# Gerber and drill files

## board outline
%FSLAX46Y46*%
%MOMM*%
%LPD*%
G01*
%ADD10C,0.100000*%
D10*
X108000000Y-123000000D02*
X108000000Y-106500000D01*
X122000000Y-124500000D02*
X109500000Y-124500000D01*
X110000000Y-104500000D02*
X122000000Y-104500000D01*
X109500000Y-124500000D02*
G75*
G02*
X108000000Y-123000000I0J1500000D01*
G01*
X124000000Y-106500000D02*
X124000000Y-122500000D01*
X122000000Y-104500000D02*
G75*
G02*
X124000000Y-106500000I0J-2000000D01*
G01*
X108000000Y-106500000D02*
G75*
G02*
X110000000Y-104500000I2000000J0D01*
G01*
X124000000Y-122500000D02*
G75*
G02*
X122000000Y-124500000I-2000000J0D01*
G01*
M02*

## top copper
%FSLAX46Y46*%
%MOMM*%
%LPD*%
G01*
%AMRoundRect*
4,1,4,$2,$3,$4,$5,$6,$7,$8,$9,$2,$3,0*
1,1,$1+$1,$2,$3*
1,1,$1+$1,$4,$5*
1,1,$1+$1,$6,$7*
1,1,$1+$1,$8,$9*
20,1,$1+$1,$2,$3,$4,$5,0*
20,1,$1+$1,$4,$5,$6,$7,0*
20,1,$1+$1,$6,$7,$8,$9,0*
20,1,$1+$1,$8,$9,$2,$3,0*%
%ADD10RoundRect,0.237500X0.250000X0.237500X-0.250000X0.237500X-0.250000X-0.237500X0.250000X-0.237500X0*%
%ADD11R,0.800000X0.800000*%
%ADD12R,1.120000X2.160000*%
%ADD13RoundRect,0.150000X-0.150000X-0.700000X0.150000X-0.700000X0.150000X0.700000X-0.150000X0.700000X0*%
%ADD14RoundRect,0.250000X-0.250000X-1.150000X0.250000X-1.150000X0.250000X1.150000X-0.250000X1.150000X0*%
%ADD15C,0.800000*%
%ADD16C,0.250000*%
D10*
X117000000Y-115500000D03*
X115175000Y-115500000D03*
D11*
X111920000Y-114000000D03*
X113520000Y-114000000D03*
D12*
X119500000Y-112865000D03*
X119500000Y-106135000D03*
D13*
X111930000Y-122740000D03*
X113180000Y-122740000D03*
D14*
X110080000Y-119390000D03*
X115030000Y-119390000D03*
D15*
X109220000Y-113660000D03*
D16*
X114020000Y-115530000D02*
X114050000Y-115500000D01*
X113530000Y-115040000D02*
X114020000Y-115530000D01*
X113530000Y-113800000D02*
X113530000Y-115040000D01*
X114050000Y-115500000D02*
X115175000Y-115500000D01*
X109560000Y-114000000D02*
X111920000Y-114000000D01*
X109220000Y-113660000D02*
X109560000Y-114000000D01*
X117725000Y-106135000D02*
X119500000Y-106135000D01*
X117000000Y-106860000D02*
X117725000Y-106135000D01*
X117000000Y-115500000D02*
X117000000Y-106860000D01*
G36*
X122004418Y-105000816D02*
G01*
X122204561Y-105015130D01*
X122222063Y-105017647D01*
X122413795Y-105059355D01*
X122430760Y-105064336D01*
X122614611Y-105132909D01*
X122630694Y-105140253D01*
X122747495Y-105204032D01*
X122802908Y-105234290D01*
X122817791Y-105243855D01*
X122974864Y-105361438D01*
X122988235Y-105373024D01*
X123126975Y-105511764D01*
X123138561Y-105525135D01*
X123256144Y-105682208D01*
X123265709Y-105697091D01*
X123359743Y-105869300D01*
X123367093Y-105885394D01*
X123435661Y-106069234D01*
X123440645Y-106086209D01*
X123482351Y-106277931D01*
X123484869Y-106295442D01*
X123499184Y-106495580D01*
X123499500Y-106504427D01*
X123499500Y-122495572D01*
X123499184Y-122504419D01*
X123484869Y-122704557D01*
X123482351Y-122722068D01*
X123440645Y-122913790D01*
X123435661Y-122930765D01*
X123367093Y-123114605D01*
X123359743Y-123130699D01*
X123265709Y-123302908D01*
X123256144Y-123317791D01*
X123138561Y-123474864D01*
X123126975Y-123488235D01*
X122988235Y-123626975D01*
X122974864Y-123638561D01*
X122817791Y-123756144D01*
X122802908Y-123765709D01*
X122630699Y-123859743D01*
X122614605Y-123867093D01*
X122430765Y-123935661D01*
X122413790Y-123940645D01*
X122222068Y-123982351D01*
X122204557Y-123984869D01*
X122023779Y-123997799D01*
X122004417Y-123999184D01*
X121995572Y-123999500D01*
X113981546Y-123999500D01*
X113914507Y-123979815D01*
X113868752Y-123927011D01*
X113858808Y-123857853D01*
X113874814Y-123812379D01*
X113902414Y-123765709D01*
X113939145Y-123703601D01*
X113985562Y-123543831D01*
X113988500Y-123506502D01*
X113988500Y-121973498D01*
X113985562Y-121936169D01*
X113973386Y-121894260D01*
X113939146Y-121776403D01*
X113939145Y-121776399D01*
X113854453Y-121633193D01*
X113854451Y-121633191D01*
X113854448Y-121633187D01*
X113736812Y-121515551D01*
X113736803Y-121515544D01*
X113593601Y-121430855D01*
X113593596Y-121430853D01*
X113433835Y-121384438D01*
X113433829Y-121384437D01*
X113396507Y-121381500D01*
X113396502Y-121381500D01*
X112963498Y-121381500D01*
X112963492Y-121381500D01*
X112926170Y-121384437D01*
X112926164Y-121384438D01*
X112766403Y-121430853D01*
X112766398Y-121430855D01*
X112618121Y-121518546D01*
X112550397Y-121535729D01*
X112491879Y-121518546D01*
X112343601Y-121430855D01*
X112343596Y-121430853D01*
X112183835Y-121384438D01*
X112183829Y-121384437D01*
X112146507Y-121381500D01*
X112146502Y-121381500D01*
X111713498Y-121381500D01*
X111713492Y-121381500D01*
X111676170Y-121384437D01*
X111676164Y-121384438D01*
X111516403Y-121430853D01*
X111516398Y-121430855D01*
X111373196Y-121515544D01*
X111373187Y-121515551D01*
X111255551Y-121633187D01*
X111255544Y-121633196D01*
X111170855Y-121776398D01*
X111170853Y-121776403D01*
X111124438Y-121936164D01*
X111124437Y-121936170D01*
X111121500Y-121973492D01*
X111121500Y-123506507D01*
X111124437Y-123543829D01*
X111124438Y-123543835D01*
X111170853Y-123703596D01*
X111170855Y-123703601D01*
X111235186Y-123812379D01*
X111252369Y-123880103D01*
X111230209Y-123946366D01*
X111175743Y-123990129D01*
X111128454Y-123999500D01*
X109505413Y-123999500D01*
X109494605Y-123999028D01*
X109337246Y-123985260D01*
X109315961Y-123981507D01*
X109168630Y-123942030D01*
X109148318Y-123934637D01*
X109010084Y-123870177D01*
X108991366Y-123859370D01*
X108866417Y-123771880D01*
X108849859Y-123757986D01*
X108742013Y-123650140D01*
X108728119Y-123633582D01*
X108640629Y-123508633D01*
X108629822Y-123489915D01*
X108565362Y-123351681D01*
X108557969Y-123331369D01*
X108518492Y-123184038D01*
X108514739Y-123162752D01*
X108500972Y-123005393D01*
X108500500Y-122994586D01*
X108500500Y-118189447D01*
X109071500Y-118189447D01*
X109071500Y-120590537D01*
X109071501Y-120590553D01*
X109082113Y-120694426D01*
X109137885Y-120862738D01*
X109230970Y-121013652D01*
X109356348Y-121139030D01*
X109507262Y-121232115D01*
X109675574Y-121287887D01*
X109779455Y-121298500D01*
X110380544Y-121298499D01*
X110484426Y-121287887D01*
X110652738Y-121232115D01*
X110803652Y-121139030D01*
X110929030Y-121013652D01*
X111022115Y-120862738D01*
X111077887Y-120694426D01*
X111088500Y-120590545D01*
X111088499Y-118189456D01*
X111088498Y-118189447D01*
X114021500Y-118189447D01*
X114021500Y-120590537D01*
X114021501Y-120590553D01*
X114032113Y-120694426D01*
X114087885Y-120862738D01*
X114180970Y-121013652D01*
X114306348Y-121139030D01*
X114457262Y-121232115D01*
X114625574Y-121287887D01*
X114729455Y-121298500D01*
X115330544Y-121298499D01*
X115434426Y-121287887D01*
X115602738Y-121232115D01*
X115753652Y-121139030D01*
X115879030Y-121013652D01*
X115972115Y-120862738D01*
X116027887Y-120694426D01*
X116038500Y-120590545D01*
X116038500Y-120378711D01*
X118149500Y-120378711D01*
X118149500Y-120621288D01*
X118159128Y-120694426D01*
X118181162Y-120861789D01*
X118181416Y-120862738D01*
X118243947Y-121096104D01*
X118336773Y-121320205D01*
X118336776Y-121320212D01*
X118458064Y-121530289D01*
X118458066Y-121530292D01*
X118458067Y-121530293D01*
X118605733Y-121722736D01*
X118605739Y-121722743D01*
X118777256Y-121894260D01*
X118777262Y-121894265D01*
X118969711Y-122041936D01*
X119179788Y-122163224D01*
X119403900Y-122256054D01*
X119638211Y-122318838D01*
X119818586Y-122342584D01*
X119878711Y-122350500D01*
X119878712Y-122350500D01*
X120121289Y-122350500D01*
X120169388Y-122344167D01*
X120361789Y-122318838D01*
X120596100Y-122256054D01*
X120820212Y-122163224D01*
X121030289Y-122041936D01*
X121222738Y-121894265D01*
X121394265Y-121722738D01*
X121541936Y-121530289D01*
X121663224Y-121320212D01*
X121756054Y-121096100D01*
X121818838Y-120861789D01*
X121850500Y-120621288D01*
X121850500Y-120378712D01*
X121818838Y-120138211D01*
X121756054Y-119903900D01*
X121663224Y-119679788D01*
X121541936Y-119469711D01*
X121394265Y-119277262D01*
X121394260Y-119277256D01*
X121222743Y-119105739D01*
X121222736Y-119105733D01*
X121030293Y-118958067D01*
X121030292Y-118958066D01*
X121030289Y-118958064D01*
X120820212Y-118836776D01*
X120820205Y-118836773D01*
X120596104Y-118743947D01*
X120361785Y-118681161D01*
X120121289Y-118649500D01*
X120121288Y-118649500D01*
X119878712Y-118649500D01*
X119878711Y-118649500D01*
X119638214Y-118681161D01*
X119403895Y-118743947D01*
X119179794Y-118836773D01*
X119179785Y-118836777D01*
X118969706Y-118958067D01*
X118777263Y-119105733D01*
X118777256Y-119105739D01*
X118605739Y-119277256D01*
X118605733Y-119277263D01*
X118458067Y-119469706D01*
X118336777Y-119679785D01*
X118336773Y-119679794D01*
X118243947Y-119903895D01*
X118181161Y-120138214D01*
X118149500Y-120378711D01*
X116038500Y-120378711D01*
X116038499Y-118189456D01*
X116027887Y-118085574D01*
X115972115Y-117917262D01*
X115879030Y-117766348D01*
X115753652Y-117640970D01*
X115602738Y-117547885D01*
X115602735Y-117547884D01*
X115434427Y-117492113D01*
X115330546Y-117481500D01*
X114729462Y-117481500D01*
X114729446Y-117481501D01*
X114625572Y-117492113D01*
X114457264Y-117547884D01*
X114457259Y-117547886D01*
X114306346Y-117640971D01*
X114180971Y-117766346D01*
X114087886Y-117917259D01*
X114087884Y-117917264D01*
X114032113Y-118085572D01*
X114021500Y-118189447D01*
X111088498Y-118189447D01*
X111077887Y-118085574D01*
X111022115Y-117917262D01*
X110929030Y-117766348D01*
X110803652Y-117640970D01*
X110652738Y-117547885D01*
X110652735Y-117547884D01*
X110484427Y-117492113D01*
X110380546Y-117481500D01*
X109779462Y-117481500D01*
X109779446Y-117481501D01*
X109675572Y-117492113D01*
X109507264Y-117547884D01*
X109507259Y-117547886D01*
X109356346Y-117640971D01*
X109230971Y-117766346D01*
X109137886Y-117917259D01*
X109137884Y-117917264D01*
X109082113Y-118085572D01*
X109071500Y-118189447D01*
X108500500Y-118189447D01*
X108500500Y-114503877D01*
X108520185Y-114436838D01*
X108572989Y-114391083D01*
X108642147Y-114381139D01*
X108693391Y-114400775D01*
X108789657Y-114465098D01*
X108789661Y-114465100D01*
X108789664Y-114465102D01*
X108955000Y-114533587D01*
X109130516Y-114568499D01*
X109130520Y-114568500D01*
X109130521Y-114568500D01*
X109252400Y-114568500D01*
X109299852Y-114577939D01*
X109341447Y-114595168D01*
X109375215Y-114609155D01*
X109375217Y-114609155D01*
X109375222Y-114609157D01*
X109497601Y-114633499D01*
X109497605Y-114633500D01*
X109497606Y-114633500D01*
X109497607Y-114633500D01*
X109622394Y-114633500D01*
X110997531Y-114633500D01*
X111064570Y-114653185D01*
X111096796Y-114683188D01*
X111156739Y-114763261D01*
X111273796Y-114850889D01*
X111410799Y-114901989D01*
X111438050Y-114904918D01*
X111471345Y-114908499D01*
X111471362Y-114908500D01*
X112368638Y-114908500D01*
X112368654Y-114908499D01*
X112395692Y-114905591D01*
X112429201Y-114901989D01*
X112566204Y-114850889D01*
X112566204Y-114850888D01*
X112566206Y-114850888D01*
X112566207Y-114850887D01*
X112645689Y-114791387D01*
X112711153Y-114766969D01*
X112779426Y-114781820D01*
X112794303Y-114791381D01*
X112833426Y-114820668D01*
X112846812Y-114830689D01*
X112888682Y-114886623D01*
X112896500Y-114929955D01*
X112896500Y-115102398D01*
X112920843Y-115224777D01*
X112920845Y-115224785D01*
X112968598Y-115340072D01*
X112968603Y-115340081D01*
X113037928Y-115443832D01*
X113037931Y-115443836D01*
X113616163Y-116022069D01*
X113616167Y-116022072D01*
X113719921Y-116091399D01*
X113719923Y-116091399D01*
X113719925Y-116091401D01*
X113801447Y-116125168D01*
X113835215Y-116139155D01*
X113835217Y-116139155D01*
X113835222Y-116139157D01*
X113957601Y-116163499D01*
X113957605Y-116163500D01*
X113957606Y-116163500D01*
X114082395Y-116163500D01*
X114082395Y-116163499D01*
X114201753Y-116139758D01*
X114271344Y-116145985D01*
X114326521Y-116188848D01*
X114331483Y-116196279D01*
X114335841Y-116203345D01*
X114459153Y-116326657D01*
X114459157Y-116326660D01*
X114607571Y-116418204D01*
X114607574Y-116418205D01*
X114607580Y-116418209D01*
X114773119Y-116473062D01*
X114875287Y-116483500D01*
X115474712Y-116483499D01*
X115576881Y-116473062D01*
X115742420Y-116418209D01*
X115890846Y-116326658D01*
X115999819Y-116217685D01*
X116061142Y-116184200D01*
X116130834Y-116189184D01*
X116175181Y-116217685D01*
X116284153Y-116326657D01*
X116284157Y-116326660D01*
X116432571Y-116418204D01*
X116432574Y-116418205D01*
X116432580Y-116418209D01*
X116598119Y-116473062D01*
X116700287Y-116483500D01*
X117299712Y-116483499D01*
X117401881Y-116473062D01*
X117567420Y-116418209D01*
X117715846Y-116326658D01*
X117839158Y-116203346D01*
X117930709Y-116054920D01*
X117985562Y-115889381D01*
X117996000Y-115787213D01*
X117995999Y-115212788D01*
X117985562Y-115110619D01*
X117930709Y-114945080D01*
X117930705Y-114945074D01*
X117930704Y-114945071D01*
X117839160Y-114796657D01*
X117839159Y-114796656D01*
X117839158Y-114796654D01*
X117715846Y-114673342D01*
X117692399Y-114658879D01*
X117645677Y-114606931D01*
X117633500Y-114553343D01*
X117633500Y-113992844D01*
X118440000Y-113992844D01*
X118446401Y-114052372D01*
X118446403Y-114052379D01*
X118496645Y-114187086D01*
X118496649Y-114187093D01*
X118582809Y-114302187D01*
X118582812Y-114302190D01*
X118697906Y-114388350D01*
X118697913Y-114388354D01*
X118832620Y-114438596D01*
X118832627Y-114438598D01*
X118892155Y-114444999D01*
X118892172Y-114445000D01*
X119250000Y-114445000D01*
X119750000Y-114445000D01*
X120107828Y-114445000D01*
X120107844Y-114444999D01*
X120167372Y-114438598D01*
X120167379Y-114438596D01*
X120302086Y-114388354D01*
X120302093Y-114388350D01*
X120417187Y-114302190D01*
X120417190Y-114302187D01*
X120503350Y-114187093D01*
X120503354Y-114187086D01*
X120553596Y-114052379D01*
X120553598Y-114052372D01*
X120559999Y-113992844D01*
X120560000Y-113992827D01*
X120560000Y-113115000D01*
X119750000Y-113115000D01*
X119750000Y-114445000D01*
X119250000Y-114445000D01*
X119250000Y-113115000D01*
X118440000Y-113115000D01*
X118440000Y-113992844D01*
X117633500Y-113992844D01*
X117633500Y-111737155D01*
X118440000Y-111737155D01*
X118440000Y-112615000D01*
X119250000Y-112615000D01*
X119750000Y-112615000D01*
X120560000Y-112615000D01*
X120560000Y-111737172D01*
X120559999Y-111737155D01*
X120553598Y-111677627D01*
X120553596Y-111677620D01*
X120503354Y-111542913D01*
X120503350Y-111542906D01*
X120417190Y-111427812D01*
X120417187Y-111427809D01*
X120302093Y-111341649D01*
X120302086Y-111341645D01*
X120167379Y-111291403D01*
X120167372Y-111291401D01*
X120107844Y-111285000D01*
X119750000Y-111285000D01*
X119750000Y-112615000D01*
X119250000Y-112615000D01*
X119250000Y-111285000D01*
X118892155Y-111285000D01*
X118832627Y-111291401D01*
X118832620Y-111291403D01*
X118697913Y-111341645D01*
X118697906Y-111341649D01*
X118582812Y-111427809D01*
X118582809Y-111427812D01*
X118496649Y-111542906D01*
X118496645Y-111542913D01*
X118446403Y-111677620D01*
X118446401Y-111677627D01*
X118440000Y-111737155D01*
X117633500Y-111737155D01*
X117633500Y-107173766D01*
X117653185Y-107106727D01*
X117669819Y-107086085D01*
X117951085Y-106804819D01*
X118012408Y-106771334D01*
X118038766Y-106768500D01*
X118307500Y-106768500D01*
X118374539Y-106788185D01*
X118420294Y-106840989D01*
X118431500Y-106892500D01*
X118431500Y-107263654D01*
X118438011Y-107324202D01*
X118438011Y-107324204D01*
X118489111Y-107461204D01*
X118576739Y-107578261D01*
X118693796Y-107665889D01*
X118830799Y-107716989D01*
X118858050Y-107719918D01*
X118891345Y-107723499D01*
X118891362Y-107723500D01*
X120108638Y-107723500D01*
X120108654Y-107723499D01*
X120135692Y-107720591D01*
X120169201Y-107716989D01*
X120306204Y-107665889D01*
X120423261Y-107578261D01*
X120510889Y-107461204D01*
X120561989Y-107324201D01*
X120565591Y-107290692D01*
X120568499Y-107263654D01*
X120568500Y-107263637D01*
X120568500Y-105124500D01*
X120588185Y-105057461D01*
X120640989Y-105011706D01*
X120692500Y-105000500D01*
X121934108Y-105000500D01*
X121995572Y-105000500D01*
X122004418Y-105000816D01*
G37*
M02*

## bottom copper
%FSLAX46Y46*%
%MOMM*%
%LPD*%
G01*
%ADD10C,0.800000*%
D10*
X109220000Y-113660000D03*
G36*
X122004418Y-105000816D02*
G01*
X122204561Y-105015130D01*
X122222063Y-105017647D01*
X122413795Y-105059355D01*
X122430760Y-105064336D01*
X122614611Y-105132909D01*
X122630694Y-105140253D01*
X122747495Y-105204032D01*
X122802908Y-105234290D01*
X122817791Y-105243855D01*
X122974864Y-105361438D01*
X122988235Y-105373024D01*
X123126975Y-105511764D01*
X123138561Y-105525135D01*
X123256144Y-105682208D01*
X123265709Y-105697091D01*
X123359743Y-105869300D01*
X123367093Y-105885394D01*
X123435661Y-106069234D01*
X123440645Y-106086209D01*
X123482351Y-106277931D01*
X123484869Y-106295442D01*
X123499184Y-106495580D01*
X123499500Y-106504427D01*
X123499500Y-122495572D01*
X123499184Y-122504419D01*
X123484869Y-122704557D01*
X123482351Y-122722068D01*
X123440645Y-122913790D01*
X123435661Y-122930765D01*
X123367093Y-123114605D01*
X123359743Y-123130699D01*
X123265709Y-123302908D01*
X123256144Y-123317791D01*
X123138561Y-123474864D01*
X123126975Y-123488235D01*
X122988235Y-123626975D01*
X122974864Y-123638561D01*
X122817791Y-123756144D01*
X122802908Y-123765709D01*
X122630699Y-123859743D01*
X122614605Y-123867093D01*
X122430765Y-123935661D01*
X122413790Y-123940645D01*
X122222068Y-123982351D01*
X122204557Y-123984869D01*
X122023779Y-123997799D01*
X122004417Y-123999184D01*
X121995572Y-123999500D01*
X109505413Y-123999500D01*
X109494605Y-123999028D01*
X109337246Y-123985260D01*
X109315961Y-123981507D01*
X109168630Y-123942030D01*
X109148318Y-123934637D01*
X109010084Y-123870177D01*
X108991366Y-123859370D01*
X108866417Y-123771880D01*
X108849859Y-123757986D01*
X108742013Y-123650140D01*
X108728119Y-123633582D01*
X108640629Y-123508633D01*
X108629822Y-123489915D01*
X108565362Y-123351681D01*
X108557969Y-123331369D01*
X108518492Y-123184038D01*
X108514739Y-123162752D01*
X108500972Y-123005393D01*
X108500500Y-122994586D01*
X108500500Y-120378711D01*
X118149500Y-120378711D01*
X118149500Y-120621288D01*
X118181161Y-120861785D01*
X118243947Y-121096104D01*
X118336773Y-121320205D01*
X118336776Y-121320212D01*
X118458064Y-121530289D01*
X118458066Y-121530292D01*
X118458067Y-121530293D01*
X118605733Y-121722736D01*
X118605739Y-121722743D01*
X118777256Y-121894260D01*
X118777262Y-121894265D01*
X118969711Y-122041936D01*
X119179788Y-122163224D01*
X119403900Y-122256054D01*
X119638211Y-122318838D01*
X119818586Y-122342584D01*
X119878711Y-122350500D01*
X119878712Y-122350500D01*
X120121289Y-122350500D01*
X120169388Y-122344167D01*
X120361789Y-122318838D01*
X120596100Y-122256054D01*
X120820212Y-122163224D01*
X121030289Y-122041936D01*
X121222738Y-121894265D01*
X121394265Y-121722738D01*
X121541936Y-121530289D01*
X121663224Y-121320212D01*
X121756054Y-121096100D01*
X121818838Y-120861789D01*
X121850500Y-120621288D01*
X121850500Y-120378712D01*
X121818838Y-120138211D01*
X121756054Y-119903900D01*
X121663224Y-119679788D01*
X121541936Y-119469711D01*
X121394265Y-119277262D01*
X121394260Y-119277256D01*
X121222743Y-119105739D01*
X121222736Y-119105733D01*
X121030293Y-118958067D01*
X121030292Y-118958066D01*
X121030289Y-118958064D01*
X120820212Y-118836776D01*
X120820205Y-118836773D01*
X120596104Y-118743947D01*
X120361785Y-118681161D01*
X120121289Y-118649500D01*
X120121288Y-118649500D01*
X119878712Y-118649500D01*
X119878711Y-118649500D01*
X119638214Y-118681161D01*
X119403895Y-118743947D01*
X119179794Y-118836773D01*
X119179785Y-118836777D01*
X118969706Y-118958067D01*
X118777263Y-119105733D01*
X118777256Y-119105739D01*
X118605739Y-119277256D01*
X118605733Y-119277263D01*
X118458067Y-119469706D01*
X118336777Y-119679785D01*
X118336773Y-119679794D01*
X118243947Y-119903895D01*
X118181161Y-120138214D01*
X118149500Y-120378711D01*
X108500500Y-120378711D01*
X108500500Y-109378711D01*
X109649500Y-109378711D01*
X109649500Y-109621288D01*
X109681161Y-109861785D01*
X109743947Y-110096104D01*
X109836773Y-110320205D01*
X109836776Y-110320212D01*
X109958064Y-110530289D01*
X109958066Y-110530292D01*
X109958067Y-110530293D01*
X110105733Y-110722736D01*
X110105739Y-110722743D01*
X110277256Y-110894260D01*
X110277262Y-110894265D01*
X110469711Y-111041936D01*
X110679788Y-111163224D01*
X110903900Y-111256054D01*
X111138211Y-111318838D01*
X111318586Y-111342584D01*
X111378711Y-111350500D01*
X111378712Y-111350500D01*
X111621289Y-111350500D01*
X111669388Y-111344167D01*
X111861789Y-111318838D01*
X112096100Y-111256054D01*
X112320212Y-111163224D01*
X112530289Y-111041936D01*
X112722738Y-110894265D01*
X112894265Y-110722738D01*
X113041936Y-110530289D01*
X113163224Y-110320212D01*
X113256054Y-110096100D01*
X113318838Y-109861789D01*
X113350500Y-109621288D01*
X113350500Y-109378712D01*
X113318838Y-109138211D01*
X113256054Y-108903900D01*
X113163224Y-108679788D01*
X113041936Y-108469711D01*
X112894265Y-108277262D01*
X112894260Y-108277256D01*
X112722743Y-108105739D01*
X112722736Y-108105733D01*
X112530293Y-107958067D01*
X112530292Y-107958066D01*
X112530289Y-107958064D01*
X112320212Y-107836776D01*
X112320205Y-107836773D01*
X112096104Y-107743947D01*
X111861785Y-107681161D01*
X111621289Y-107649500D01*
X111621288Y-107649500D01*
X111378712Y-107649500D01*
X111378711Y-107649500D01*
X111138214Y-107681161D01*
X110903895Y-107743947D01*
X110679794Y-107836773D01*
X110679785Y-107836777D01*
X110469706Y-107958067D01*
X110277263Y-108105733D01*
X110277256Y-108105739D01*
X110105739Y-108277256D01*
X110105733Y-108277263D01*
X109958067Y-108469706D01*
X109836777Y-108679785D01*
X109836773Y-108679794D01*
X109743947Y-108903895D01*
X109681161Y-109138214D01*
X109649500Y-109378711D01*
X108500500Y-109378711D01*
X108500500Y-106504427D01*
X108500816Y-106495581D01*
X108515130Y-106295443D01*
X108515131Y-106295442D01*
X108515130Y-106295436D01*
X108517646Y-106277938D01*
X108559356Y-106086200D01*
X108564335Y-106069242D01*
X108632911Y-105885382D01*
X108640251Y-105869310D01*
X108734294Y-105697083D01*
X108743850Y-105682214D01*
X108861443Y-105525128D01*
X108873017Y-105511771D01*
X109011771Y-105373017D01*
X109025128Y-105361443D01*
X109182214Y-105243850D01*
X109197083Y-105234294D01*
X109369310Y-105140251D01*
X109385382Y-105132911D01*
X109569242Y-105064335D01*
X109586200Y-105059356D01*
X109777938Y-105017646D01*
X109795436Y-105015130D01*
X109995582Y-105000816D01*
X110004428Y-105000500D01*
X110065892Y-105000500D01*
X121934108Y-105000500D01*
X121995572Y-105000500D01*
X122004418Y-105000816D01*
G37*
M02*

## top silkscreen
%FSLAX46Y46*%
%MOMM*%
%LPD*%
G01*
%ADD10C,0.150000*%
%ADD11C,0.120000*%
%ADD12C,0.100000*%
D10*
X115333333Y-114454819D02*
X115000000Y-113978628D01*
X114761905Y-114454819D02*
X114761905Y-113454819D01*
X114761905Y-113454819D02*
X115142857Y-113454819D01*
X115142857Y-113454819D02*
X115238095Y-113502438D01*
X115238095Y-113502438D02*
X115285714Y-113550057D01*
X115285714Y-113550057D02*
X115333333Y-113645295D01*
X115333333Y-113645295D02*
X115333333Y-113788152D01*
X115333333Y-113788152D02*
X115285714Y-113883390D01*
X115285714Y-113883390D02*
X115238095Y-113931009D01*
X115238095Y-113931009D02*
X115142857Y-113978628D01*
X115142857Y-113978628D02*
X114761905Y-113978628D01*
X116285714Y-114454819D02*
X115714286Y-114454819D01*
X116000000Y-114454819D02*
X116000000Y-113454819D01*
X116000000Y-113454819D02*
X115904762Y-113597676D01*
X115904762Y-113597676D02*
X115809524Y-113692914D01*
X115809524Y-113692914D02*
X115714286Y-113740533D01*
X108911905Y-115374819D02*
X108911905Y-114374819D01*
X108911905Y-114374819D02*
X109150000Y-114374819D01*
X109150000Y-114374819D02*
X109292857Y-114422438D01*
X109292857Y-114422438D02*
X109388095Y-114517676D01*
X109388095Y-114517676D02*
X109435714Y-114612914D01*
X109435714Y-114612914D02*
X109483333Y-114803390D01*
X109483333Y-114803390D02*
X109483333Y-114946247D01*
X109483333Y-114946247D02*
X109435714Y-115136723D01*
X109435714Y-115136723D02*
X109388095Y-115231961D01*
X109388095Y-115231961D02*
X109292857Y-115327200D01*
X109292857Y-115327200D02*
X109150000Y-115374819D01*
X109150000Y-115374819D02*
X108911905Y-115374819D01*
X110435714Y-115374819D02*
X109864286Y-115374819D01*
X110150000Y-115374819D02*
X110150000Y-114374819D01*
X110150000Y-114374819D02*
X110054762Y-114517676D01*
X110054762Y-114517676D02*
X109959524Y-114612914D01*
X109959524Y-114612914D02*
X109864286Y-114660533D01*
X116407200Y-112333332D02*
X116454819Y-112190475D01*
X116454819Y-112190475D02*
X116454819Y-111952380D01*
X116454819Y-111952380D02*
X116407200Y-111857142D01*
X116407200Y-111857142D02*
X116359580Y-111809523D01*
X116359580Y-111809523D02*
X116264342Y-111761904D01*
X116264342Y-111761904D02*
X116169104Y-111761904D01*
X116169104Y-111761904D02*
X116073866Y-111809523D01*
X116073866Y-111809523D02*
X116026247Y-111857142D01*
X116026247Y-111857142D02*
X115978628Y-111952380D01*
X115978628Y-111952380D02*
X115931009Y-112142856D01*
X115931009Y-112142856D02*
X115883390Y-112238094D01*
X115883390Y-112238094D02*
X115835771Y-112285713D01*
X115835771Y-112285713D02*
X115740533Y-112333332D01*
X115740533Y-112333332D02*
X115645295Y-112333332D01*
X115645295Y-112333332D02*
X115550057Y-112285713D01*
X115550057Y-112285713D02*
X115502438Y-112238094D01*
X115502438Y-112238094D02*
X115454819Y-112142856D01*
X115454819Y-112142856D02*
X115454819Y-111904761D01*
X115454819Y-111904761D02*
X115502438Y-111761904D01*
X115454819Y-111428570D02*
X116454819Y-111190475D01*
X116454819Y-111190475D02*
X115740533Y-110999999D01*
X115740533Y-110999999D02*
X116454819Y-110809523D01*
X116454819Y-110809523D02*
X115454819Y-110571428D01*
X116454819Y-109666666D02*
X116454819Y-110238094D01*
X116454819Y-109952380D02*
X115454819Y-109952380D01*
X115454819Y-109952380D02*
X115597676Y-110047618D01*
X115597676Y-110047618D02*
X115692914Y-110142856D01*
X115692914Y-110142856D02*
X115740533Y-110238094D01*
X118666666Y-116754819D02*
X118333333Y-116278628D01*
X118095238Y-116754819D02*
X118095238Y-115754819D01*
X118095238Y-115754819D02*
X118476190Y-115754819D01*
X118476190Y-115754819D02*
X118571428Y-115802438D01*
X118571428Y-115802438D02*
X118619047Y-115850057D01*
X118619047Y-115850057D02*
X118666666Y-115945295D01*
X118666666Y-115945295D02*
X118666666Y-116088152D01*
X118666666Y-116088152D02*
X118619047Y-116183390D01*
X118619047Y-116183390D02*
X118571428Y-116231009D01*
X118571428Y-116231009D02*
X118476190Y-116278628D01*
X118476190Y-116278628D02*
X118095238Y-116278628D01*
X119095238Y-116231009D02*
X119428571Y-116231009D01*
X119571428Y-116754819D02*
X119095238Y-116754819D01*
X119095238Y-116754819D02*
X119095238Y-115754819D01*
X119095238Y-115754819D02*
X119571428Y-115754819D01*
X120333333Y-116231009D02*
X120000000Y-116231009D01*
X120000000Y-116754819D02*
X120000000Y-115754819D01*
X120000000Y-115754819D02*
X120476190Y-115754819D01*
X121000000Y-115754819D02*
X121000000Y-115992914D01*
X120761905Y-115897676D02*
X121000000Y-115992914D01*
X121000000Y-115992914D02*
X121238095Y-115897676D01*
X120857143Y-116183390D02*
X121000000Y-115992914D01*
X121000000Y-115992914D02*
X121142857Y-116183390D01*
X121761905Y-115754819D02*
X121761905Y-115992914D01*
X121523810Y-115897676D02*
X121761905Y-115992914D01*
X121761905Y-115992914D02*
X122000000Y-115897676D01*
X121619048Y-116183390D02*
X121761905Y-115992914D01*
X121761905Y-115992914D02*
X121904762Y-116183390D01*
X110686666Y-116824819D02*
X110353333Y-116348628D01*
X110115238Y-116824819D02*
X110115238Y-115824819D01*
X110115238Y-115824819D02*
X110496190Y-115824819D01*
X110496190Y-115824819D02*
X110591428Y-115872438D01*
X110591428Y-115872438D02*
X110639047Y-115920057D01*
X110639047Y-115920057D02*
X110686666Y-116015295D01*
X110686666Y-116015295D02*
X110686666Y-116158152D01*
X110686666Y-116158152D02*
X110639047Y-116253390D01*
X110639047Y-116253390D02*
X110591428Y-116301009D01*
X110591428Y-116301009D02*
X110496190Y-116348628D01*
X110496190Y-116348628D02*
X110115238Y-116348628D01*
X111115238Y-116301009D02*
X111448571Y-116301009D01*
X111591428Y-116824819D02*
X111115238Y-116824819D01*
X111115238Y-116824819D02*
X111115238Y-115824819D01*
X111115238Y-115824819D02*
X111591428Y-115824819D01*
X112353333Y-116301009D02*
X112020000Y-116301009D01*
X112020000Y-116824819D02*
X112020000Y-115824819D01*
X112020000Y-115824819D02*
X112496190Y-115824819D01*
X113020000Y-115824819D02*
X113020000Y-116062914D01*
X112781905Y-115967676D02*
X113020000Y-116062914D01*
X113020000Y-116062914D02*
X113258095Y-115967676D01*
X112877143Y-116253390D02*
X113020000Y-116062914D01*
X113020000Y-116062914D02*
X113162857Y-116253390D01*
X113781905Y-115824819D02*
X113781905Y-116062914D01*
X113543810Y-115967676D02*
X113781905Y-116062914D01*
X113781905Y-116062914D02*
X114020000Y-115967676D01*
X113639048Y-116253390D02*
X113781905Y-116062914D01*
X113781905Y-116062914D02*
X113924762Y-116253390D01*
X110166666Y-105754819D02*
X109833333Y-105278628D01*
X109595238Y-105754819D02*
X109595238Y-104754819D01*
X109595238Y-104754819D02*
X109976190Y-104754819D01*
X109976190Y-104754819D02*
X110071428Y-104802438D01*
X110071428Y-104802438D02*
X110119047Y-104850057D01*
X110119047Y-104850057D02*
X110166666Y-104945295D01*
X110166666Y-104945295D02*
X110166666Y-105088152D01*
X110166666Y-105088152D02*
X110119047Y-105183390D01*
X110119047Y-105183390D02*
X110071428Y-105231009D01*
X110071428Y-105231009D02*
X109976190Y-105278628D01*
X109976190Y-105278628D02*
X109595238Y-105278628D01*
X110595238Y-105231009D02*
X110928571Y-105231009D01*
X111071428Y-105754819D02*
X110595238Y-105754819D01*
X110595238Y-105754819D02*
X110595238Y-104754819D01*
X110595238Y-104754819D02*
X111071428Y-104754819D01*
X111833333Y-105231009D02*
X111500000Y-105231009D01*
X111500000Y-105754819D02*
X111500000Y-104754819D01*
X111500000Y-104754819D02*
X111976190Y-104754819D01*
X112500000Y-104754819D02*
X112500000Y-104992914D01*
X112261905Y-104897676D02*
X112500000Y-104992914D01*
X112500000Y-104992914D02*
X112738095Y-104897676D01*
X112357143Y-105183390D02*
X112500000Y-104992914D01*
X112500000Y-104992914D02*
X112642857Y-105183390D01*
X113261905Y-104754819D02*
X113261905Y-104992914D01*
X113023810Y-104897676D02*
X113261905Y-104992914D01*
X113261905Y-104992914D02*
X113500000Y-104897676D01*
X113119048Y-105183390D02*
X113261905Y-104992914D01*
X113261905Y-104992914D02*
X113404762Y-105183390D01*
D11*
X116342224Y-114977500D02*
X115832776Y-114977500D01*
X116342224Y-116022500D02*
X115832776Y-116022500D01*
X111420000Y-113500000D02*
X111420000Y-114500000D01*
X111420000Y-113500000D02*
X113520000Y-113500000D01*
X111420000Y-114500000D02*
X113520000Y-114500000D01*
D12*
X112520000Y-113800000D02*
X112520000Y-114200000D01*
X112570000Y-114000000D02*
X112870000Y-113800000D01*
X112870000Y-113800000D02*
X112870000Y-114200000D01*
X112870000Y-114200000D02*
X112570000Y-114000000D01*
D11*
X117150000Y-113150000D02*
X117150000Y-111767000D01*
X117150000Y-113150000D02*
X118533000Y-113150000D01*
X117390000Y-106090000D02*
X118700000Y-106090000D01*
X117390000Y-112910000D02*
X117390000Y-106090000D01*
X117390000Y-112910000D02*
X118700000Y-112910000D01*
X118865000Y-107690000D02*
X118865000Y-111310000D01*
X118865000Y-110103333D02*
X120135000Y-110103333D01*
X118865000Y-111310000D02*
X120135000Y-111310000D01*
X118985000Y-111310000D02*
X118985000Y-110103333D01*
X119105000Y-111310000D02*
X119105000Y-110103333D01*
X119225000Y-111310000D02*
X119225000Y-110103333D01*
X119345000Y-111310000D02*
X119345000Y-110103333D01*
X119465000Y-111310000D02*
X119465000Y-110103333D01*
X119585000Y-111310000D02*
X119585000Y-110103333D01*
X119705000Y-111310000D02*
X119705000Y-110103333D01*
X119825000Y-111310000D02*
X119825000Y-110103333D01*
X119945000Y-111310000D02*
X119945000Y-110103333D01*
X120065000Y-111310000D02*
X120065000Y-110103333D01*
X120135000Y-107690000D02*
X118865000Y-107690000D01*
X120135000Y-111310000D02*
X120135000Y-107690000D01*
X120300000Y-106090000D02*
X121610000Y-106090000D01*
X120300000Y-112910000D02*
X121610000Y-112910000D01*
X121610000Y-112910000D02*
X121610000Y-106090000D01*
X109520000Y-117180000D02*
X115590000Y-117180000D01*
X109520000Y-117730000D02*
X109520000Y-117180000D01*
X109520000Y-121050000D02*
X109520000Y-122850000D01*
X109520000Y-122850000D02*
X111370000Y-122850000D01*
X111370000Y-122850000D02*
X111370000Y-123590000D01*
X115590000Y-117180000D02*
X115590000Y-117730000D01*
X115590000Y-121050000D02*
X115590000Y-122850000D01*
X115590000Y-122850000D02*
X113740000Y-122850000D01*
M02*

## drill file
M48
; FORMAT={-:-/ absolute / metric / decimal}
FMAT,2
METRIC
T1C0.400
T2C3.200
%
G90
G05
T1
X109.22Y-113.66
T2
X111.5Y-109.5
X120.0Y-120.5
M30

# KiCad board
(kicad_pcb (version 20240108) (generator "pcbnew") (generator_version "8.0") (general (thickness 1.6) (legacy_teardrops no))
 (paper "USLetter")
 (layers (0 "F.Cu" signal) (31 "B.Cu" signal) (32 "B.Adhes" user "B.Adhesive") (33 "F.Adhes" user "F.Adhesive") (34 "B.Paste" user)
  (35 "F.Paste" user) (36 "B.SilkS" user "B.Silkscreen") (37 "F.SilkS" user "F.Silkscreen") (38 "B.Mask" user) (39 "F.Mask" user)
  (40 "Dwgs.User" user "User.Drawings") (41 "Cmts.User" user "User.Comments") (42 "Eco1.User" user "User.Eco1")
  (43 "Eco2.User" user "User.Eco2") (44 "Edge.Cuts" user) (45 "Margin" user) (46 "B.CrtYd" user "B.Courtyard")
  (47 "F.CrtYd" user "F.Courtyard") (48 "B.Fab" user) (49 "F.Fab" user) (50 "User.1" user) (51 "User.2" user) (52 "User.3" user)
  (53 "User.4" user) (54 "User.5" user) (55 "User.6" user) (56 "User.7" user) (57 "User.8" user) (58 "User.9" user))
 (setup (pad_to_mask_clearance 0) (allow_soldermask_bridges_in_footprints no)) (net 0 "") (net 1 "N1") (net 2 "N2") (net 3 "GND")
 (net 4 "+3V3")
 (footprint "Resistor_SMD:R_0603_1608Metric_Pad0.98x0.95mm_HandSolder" (layer "F.Cu") (at 116.0875 115.5 180)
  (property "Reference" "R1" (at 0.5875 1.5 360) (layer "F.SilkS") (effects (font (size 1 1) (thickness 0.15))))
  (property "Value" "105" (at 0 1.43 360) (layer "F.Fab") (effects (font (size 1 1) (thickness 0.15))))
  (fp_line (start -0.254724 0.5225) (end 0.254724 0.5225) (stroke (width 0.12) (type solid)) (layer "F.SilkS"))
  (fp_line (start -0.254724 -0.5225) (end 0.254724 -0.5225) (stroke (width 0.12) (type solid)) (layer "F.SilkS"))
  (pad "1" smd roundrect (at -0.9125 0 180) (size 0.975 0.95) (layers "F.Cu" "F.Paste" "F.Mask") (roundrect_rratio 0.25) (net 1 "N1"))
  (pad "2" smd roundrect (at 0.9125 0 180) (size 0.975 0.95) (layers "F.Cu" "F.Paste" "F.Mask") (roundrect_rratio 0.25) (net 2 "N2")))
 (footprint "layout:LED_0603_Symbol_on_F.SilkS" (layer "F.Cu") (at 112.72 114)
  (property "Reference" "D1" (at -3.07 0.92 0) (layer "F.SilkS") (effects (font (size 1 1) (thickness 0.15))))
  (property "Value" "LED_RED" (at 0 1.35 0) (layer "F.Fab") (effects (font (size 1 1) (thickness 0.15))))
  (fp_line (start -1.3 -0.5) (end -1.3 0.5) (stroke (width 0.12) (type solid)) (layer "F.SilkS"))
  (fp_line (start -1.3 -0.5) (end 0.8 -0.5) (stroke (width 0.12) (type solid)) (layer "F.SilkS"))
  (fp_line (start -1.3 0.5) (end 0.8 0.5) (stroke (width 0.12) (type solid)) (layer "F.SilkS"))
  (fp_line (start -0.2 -0.2) (end -0.2 0.2) (stroke (width 0.1) (type solid)) (layer "F.SilkS"))
  (fp_line (start -0.15 0) (end 0.15 -0.2) (stroke (width 0.1) (type solid)) (layer "F.SilkS"))
  (fp_line (start 0.15 -0.2) (end 0.15 0.2) (stroke (width 0.1) (type solid)) (layer "F.SilkS"))
  (fp_line (start 0.15 0.2) (end -0.15 0) (stroke (width 0.1) (type solid)) (layer "F.SilkS"))
  (pad "1" smd rect (at -0.8 0 180) (size 0.8 0.8) (layers "F.Cu" "F.Paste" "F.Mask") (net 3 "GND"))
  (pad "2" smd rect (at 0.8 0 180) (size 0.8 0.8) (layers "F.Cu" "F.Paste" "F.Mask") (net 2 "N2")))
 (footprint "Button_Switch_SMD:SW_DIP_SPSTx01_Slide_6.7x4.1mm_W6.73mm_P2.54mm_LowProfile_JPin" (layer "F.Cu") (at 119.5 109.5 90)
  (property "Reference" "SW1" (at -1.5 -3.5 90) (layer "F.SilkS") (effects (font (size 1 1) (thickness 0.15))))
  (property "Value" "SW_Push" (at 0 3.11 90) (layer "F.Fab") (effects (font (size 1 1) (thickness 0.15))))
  (fp_line (start -3.65 -2.35) (end -2.267 -2.35) (stroke (width 0.12) (type solid)) (layer "F.SilkS"))
  (fp_line (start -3.65 -2.35) (end -3.65 -0.967) (stroke (width 0.12) (type solid)) (layer "F.SilkS"))
  (fp_line (start 3.41 -2.11) (end 3.41 -0.8) (stroke (width 0.12) (type solid)) (layer "F.SilkS"))
  (fp_line (start -3.41 -2.11) (end 3.41 -2.11) (stroke (width 0.12) (type solid)) (layer "F.SilkS"))
  (fp_line (start -3.41 -2.11) (end -3.41 -0.8) (stroke (width 0.12) (type solid)) (layer "F.SilkS"))
  (fp_line (start 1.81 -0.635) (end -1.81 -0.635) (stroke (width 0.12) (type solid)) (layer "F.SilkS"))
  (fp_line (start -0.603333 -0.635) (end -0.603333 0.635) (stroke (width 0.12) (type solid)) (layer "F.SilkS"))
  (fp_line (start -1.81 -0.635) (end -1.81 0.635) (stroke (width 0.12) (type solid)) (layer "F.SilkS"))
  (fp_line (start -1.81 -0.515) (end -0.603333 -0.515) (stroke (width 0.12) (type solid)) (layer "F.SilkS"))
  (fp_line (start -1.81 -0.395) (end -0.603333 -0.395) (stroke (width 0.12) (type solid)) (layer "F.SilkS"))
  (fp_line (start -1.81 -0.275) (end -0.603333 -0.275) (stroke (width 0.12) (type solid)) (layer "F.SilkS"))
  (fp_line (start -1.81 -0.155) (end -0.603333 -0.155) (stroke (width 0.12) (type solid)) (layer "F.SilkS"))
  (fp_line (start -1.81 -0.035) (end -0.603333 -0.035) (stroke (width 0.12) (type solid)) (layer "F.SilkS"))
  (fp_line (start -1.81 0.085) (end -0.603333 0.085) (stroke (width 0.12) (type solid)) (layer "F.SilkS"))
  (fp_line (start -1.81 0.205) (end -0.603333 0.205) (stroke (width 0.12) (type solid)) (layer "F.SilkS"))
  (fp_line (start -1.81 0.325) (end -0.603333 0.325) (stroke (width 0.12) (type solid)) (layer "F.SilkS"))
  (fp_line (start -1.81 0.445) (end -0.603333 0.445) (stroke (width 0.12) (type solid)) (layer "F.SilkS"))
  (fp_line (start -1.81 0.565) (end -0.603333 0.565) (stroke (width 0.12) (type solid)) (layer "F.SilkS"))
  (fp_line (start 1.81 0.635) (end 1.81 -0.635) (stroke (width 0.12) (type solid)) (layer "F.SilkS"))
  (fp_line (start -1.81 0.635) (end 1.81 0.635) (stroke (width 0.12) (type solid)) (layer "F.SilkS"))
  (fp_line (start 3.41 0.8) (end 3.41 2.11) (stroke (width 0.12) (type solid)) (layer "F.SilkS"))
  (fp_line (start -3.41 0.8) (end -3.41 2.11) (stroke (width 0.12) (type solid)) (layer "F.SilkS"))
  (fp_line (start -3.41 2.11) (end 3.41 2.11) (stroke (width 0.12) (type solid)) (layer "F.SilkS"))
  (pad "1" smd rect (at -3.365 0 90) (size 2.16 1.12) (layers "F.Cu" "F.Paste" "F.Mask") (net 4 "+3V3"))
  (pad "2" smd rect (at 3.365 0 90) (size 2.16 1.12) (layers "F.Cu" "F.Paste" "F.Mask") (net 1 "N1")))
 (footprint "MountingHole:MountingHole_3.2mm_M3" (layer "F.Cu") (at 120 120.5)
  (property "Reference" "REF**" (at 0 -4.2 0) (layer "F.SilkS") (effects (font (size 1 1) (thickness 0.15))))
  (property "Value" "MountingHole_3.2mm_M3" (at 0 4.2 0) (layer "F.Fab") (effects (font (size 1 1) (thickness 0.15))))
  (pad "" np_thru_hole circle (at 0 0) (size 3.2 3.2) (drill 3.2) (layers "*.Cu" "*.Mask")))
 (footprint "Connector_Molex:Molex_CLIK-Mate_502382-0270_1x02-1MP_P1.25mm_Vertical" (layer "F.Cu") (at 112.555 120.79)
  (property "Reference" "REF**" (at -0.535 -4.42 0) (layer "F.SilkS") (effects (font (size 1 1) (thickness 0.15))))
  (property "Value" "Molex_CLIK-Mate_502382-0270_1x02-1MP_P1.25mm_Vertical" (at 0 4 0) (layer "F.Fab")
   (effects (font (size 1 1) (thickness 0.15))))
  (fp_line (start -3.035 -3.61) (end 3.035 -3.61) (stroke (width 0.12) (type solid)) (layer "F.SilkS"))
  (fp_line (start -3.035 -3.06) (end -3.035 -3.61) (stroke (width 0.12) (type solid)) (layer "F.SilkS"))
  (fp_line (start -3.035 0.26) (end -3.035 2.06) (stroke (width 0.12) (type solid)) (layer "F.SilkS"))
  (fp_line (start -3.035 2.06) (end -1.185 2.06) (stroke (width 0.12) (type solid)) (layer "F.SilkS"))
  (fp_line (start -1.185 2.06) (end -1.185 2.8) (stroke (width 0.12) (type solid)) (layer "F.SilkS"))
  (fp_line (start 3.035 -3.61) (end 3.035 -3.06) (stroke (width 0.12) (type solid)) (layer "F.SilkS"))
  (fp_line (start 3.035 0.26) (end 3.035 2.06) (stroke (width 0.12) (type solid)) (layer "F.SilkS"))
  (fp_line (start 3.035 2.06) (end 1.185 2.06) (stroke (width 0.12) (type solid)) (layer "F.SilkS"))
  (pad "1" smd roundrect (at -0.625 1.95) (size 0.6 1.7) (layers "F.Cu" "F.Paste" "F.Mask") (roundrect_rratio 0.25))
  (pad "2" smd roundrect (at 0.625 1.95) (size 0.6 1.7) (layers "F.Cu" "F.Paste" "F.Mask") (roundrect_rratio 0.25))
  (pad "MP" smd roundrect (at -2.475 -1.4) (size 1 2.8) (layers "F.Cu" "F.Paste" "F.Mask") (roundrect_rratio 0.25))
  (pad "MP" smd roundrect (at 2.475 -1.4) (size 1 2.8) (layers "F.Cu" "F.Paste" "F.Mask") (roundrect_rratio 0.25)))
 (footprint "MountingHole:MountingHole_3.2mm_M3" (layer "F.Cu") (at 111.5 109.5)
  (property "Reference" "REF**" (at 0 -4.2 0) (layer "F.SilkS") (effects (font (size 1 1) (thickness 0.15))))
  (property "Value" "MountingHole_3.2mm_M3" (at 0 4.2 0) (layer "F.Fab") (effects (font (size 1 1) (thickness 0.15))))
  (pad "" np_thru_hole circle (at 0 0) (size 3.2 3.2) (drill 3.2) (layers "*.Cu" "*.Mask")))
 (gr_line (start 108 123) (end 108 106.5) (stroke (width 0.1) (type default)) (layer "Edge.Cuts"))
 (gr_line (start 122 124.5) (end 109.5 124.5) (stroke (width 0.1) (type default)) (layer "Edge.Cuts"))
 (gr_line (start 110 104.5) (end 122 104.5) (stroke (width 0.1) (type default)) (layer "Edge.Cuts"))
 (gr_arc (start 109.5 124.5) (mid 108.43934 124.06066) (end 108 123) (stroke (width 0.1) (type default)) (layer "Edge.Cuts"))
 (gr_line (start 124 106.5) (end 124 122.5) (stroke (width 0.1) (type default)) (layer "Edge.Cuts"))
 (gr_arc (start 122 104.5) (mid 123.414214 105.085786) (end 124 106.5) (stroke (width 0.1) (type default)) (layer "Edge.Cuts"))
 (gr_arc (start 108 106.5) (mid 108.585786 105.085786) (end 110 104.5) (stroke (width 0.1) (type default)) (layer "Edge.Cuts"))
 (gr_arc (start 124 122.5) (mid 123.414214 123.914214) (end 122 124.5) (stroke (width 0.1) (type default)) (layer "Edge.Cuts"))
 (segment (start 114.02 115.53) (end 114.05 115.5) (width 0.25) (layer "F.Cu") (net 2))
 (segment (start 113.53 115.04) (end 114.02 115.53) (width 0.25) (layer "F.Cu") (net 2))
 (segment (start 113.53 113.8) (end 113.53 115.04) (width 0.25) (layer "F.Cu") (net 2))
 (segment (start 114.05 115.5) (end 115.175 115.5) (width 0.25) (layer "F.Cu") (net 2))
 (segment (start 109.56 114) (end 111.92 114) (width 0.25) (layer "F.Cu") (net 3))
 (segment (start 109.22 113.66) (end 109.56 114) (width 0.25) (layer "F.Cu") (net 3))
 (via (at 109.22 113.66) (size 0.8) (drill 0.4) (layers "F.Cu" "B.Cu") (free yes) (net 3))
 (segment (start 117.725 106.135) (end 119.5 106.135) (width 0.25) (layer "F.Cu") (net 1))
 (segment (start 117 106.86) (end 117.725 106.135) (width 0.25) (layer "F.Cu") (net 1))
 (segment (start 117 115.5) (end 117 106.86) (width 0.25) (layer "F.Cu") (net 1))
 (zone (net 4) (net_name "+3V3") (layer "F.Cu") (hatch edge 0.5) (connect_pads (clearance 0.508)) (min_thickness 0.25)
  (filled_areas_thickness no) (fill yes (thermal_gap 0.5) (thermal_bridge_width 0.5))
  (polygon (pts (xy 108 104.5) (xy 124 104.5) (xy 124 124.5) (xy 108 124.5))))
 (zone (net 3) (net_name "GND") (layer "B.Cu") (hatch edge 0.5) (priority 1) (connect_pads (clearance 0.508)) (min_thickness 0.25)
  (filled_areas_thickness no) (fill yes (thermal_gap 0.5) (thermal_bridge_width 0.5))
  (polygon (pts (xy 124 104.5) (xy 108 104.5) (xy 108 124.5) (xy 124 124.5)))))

